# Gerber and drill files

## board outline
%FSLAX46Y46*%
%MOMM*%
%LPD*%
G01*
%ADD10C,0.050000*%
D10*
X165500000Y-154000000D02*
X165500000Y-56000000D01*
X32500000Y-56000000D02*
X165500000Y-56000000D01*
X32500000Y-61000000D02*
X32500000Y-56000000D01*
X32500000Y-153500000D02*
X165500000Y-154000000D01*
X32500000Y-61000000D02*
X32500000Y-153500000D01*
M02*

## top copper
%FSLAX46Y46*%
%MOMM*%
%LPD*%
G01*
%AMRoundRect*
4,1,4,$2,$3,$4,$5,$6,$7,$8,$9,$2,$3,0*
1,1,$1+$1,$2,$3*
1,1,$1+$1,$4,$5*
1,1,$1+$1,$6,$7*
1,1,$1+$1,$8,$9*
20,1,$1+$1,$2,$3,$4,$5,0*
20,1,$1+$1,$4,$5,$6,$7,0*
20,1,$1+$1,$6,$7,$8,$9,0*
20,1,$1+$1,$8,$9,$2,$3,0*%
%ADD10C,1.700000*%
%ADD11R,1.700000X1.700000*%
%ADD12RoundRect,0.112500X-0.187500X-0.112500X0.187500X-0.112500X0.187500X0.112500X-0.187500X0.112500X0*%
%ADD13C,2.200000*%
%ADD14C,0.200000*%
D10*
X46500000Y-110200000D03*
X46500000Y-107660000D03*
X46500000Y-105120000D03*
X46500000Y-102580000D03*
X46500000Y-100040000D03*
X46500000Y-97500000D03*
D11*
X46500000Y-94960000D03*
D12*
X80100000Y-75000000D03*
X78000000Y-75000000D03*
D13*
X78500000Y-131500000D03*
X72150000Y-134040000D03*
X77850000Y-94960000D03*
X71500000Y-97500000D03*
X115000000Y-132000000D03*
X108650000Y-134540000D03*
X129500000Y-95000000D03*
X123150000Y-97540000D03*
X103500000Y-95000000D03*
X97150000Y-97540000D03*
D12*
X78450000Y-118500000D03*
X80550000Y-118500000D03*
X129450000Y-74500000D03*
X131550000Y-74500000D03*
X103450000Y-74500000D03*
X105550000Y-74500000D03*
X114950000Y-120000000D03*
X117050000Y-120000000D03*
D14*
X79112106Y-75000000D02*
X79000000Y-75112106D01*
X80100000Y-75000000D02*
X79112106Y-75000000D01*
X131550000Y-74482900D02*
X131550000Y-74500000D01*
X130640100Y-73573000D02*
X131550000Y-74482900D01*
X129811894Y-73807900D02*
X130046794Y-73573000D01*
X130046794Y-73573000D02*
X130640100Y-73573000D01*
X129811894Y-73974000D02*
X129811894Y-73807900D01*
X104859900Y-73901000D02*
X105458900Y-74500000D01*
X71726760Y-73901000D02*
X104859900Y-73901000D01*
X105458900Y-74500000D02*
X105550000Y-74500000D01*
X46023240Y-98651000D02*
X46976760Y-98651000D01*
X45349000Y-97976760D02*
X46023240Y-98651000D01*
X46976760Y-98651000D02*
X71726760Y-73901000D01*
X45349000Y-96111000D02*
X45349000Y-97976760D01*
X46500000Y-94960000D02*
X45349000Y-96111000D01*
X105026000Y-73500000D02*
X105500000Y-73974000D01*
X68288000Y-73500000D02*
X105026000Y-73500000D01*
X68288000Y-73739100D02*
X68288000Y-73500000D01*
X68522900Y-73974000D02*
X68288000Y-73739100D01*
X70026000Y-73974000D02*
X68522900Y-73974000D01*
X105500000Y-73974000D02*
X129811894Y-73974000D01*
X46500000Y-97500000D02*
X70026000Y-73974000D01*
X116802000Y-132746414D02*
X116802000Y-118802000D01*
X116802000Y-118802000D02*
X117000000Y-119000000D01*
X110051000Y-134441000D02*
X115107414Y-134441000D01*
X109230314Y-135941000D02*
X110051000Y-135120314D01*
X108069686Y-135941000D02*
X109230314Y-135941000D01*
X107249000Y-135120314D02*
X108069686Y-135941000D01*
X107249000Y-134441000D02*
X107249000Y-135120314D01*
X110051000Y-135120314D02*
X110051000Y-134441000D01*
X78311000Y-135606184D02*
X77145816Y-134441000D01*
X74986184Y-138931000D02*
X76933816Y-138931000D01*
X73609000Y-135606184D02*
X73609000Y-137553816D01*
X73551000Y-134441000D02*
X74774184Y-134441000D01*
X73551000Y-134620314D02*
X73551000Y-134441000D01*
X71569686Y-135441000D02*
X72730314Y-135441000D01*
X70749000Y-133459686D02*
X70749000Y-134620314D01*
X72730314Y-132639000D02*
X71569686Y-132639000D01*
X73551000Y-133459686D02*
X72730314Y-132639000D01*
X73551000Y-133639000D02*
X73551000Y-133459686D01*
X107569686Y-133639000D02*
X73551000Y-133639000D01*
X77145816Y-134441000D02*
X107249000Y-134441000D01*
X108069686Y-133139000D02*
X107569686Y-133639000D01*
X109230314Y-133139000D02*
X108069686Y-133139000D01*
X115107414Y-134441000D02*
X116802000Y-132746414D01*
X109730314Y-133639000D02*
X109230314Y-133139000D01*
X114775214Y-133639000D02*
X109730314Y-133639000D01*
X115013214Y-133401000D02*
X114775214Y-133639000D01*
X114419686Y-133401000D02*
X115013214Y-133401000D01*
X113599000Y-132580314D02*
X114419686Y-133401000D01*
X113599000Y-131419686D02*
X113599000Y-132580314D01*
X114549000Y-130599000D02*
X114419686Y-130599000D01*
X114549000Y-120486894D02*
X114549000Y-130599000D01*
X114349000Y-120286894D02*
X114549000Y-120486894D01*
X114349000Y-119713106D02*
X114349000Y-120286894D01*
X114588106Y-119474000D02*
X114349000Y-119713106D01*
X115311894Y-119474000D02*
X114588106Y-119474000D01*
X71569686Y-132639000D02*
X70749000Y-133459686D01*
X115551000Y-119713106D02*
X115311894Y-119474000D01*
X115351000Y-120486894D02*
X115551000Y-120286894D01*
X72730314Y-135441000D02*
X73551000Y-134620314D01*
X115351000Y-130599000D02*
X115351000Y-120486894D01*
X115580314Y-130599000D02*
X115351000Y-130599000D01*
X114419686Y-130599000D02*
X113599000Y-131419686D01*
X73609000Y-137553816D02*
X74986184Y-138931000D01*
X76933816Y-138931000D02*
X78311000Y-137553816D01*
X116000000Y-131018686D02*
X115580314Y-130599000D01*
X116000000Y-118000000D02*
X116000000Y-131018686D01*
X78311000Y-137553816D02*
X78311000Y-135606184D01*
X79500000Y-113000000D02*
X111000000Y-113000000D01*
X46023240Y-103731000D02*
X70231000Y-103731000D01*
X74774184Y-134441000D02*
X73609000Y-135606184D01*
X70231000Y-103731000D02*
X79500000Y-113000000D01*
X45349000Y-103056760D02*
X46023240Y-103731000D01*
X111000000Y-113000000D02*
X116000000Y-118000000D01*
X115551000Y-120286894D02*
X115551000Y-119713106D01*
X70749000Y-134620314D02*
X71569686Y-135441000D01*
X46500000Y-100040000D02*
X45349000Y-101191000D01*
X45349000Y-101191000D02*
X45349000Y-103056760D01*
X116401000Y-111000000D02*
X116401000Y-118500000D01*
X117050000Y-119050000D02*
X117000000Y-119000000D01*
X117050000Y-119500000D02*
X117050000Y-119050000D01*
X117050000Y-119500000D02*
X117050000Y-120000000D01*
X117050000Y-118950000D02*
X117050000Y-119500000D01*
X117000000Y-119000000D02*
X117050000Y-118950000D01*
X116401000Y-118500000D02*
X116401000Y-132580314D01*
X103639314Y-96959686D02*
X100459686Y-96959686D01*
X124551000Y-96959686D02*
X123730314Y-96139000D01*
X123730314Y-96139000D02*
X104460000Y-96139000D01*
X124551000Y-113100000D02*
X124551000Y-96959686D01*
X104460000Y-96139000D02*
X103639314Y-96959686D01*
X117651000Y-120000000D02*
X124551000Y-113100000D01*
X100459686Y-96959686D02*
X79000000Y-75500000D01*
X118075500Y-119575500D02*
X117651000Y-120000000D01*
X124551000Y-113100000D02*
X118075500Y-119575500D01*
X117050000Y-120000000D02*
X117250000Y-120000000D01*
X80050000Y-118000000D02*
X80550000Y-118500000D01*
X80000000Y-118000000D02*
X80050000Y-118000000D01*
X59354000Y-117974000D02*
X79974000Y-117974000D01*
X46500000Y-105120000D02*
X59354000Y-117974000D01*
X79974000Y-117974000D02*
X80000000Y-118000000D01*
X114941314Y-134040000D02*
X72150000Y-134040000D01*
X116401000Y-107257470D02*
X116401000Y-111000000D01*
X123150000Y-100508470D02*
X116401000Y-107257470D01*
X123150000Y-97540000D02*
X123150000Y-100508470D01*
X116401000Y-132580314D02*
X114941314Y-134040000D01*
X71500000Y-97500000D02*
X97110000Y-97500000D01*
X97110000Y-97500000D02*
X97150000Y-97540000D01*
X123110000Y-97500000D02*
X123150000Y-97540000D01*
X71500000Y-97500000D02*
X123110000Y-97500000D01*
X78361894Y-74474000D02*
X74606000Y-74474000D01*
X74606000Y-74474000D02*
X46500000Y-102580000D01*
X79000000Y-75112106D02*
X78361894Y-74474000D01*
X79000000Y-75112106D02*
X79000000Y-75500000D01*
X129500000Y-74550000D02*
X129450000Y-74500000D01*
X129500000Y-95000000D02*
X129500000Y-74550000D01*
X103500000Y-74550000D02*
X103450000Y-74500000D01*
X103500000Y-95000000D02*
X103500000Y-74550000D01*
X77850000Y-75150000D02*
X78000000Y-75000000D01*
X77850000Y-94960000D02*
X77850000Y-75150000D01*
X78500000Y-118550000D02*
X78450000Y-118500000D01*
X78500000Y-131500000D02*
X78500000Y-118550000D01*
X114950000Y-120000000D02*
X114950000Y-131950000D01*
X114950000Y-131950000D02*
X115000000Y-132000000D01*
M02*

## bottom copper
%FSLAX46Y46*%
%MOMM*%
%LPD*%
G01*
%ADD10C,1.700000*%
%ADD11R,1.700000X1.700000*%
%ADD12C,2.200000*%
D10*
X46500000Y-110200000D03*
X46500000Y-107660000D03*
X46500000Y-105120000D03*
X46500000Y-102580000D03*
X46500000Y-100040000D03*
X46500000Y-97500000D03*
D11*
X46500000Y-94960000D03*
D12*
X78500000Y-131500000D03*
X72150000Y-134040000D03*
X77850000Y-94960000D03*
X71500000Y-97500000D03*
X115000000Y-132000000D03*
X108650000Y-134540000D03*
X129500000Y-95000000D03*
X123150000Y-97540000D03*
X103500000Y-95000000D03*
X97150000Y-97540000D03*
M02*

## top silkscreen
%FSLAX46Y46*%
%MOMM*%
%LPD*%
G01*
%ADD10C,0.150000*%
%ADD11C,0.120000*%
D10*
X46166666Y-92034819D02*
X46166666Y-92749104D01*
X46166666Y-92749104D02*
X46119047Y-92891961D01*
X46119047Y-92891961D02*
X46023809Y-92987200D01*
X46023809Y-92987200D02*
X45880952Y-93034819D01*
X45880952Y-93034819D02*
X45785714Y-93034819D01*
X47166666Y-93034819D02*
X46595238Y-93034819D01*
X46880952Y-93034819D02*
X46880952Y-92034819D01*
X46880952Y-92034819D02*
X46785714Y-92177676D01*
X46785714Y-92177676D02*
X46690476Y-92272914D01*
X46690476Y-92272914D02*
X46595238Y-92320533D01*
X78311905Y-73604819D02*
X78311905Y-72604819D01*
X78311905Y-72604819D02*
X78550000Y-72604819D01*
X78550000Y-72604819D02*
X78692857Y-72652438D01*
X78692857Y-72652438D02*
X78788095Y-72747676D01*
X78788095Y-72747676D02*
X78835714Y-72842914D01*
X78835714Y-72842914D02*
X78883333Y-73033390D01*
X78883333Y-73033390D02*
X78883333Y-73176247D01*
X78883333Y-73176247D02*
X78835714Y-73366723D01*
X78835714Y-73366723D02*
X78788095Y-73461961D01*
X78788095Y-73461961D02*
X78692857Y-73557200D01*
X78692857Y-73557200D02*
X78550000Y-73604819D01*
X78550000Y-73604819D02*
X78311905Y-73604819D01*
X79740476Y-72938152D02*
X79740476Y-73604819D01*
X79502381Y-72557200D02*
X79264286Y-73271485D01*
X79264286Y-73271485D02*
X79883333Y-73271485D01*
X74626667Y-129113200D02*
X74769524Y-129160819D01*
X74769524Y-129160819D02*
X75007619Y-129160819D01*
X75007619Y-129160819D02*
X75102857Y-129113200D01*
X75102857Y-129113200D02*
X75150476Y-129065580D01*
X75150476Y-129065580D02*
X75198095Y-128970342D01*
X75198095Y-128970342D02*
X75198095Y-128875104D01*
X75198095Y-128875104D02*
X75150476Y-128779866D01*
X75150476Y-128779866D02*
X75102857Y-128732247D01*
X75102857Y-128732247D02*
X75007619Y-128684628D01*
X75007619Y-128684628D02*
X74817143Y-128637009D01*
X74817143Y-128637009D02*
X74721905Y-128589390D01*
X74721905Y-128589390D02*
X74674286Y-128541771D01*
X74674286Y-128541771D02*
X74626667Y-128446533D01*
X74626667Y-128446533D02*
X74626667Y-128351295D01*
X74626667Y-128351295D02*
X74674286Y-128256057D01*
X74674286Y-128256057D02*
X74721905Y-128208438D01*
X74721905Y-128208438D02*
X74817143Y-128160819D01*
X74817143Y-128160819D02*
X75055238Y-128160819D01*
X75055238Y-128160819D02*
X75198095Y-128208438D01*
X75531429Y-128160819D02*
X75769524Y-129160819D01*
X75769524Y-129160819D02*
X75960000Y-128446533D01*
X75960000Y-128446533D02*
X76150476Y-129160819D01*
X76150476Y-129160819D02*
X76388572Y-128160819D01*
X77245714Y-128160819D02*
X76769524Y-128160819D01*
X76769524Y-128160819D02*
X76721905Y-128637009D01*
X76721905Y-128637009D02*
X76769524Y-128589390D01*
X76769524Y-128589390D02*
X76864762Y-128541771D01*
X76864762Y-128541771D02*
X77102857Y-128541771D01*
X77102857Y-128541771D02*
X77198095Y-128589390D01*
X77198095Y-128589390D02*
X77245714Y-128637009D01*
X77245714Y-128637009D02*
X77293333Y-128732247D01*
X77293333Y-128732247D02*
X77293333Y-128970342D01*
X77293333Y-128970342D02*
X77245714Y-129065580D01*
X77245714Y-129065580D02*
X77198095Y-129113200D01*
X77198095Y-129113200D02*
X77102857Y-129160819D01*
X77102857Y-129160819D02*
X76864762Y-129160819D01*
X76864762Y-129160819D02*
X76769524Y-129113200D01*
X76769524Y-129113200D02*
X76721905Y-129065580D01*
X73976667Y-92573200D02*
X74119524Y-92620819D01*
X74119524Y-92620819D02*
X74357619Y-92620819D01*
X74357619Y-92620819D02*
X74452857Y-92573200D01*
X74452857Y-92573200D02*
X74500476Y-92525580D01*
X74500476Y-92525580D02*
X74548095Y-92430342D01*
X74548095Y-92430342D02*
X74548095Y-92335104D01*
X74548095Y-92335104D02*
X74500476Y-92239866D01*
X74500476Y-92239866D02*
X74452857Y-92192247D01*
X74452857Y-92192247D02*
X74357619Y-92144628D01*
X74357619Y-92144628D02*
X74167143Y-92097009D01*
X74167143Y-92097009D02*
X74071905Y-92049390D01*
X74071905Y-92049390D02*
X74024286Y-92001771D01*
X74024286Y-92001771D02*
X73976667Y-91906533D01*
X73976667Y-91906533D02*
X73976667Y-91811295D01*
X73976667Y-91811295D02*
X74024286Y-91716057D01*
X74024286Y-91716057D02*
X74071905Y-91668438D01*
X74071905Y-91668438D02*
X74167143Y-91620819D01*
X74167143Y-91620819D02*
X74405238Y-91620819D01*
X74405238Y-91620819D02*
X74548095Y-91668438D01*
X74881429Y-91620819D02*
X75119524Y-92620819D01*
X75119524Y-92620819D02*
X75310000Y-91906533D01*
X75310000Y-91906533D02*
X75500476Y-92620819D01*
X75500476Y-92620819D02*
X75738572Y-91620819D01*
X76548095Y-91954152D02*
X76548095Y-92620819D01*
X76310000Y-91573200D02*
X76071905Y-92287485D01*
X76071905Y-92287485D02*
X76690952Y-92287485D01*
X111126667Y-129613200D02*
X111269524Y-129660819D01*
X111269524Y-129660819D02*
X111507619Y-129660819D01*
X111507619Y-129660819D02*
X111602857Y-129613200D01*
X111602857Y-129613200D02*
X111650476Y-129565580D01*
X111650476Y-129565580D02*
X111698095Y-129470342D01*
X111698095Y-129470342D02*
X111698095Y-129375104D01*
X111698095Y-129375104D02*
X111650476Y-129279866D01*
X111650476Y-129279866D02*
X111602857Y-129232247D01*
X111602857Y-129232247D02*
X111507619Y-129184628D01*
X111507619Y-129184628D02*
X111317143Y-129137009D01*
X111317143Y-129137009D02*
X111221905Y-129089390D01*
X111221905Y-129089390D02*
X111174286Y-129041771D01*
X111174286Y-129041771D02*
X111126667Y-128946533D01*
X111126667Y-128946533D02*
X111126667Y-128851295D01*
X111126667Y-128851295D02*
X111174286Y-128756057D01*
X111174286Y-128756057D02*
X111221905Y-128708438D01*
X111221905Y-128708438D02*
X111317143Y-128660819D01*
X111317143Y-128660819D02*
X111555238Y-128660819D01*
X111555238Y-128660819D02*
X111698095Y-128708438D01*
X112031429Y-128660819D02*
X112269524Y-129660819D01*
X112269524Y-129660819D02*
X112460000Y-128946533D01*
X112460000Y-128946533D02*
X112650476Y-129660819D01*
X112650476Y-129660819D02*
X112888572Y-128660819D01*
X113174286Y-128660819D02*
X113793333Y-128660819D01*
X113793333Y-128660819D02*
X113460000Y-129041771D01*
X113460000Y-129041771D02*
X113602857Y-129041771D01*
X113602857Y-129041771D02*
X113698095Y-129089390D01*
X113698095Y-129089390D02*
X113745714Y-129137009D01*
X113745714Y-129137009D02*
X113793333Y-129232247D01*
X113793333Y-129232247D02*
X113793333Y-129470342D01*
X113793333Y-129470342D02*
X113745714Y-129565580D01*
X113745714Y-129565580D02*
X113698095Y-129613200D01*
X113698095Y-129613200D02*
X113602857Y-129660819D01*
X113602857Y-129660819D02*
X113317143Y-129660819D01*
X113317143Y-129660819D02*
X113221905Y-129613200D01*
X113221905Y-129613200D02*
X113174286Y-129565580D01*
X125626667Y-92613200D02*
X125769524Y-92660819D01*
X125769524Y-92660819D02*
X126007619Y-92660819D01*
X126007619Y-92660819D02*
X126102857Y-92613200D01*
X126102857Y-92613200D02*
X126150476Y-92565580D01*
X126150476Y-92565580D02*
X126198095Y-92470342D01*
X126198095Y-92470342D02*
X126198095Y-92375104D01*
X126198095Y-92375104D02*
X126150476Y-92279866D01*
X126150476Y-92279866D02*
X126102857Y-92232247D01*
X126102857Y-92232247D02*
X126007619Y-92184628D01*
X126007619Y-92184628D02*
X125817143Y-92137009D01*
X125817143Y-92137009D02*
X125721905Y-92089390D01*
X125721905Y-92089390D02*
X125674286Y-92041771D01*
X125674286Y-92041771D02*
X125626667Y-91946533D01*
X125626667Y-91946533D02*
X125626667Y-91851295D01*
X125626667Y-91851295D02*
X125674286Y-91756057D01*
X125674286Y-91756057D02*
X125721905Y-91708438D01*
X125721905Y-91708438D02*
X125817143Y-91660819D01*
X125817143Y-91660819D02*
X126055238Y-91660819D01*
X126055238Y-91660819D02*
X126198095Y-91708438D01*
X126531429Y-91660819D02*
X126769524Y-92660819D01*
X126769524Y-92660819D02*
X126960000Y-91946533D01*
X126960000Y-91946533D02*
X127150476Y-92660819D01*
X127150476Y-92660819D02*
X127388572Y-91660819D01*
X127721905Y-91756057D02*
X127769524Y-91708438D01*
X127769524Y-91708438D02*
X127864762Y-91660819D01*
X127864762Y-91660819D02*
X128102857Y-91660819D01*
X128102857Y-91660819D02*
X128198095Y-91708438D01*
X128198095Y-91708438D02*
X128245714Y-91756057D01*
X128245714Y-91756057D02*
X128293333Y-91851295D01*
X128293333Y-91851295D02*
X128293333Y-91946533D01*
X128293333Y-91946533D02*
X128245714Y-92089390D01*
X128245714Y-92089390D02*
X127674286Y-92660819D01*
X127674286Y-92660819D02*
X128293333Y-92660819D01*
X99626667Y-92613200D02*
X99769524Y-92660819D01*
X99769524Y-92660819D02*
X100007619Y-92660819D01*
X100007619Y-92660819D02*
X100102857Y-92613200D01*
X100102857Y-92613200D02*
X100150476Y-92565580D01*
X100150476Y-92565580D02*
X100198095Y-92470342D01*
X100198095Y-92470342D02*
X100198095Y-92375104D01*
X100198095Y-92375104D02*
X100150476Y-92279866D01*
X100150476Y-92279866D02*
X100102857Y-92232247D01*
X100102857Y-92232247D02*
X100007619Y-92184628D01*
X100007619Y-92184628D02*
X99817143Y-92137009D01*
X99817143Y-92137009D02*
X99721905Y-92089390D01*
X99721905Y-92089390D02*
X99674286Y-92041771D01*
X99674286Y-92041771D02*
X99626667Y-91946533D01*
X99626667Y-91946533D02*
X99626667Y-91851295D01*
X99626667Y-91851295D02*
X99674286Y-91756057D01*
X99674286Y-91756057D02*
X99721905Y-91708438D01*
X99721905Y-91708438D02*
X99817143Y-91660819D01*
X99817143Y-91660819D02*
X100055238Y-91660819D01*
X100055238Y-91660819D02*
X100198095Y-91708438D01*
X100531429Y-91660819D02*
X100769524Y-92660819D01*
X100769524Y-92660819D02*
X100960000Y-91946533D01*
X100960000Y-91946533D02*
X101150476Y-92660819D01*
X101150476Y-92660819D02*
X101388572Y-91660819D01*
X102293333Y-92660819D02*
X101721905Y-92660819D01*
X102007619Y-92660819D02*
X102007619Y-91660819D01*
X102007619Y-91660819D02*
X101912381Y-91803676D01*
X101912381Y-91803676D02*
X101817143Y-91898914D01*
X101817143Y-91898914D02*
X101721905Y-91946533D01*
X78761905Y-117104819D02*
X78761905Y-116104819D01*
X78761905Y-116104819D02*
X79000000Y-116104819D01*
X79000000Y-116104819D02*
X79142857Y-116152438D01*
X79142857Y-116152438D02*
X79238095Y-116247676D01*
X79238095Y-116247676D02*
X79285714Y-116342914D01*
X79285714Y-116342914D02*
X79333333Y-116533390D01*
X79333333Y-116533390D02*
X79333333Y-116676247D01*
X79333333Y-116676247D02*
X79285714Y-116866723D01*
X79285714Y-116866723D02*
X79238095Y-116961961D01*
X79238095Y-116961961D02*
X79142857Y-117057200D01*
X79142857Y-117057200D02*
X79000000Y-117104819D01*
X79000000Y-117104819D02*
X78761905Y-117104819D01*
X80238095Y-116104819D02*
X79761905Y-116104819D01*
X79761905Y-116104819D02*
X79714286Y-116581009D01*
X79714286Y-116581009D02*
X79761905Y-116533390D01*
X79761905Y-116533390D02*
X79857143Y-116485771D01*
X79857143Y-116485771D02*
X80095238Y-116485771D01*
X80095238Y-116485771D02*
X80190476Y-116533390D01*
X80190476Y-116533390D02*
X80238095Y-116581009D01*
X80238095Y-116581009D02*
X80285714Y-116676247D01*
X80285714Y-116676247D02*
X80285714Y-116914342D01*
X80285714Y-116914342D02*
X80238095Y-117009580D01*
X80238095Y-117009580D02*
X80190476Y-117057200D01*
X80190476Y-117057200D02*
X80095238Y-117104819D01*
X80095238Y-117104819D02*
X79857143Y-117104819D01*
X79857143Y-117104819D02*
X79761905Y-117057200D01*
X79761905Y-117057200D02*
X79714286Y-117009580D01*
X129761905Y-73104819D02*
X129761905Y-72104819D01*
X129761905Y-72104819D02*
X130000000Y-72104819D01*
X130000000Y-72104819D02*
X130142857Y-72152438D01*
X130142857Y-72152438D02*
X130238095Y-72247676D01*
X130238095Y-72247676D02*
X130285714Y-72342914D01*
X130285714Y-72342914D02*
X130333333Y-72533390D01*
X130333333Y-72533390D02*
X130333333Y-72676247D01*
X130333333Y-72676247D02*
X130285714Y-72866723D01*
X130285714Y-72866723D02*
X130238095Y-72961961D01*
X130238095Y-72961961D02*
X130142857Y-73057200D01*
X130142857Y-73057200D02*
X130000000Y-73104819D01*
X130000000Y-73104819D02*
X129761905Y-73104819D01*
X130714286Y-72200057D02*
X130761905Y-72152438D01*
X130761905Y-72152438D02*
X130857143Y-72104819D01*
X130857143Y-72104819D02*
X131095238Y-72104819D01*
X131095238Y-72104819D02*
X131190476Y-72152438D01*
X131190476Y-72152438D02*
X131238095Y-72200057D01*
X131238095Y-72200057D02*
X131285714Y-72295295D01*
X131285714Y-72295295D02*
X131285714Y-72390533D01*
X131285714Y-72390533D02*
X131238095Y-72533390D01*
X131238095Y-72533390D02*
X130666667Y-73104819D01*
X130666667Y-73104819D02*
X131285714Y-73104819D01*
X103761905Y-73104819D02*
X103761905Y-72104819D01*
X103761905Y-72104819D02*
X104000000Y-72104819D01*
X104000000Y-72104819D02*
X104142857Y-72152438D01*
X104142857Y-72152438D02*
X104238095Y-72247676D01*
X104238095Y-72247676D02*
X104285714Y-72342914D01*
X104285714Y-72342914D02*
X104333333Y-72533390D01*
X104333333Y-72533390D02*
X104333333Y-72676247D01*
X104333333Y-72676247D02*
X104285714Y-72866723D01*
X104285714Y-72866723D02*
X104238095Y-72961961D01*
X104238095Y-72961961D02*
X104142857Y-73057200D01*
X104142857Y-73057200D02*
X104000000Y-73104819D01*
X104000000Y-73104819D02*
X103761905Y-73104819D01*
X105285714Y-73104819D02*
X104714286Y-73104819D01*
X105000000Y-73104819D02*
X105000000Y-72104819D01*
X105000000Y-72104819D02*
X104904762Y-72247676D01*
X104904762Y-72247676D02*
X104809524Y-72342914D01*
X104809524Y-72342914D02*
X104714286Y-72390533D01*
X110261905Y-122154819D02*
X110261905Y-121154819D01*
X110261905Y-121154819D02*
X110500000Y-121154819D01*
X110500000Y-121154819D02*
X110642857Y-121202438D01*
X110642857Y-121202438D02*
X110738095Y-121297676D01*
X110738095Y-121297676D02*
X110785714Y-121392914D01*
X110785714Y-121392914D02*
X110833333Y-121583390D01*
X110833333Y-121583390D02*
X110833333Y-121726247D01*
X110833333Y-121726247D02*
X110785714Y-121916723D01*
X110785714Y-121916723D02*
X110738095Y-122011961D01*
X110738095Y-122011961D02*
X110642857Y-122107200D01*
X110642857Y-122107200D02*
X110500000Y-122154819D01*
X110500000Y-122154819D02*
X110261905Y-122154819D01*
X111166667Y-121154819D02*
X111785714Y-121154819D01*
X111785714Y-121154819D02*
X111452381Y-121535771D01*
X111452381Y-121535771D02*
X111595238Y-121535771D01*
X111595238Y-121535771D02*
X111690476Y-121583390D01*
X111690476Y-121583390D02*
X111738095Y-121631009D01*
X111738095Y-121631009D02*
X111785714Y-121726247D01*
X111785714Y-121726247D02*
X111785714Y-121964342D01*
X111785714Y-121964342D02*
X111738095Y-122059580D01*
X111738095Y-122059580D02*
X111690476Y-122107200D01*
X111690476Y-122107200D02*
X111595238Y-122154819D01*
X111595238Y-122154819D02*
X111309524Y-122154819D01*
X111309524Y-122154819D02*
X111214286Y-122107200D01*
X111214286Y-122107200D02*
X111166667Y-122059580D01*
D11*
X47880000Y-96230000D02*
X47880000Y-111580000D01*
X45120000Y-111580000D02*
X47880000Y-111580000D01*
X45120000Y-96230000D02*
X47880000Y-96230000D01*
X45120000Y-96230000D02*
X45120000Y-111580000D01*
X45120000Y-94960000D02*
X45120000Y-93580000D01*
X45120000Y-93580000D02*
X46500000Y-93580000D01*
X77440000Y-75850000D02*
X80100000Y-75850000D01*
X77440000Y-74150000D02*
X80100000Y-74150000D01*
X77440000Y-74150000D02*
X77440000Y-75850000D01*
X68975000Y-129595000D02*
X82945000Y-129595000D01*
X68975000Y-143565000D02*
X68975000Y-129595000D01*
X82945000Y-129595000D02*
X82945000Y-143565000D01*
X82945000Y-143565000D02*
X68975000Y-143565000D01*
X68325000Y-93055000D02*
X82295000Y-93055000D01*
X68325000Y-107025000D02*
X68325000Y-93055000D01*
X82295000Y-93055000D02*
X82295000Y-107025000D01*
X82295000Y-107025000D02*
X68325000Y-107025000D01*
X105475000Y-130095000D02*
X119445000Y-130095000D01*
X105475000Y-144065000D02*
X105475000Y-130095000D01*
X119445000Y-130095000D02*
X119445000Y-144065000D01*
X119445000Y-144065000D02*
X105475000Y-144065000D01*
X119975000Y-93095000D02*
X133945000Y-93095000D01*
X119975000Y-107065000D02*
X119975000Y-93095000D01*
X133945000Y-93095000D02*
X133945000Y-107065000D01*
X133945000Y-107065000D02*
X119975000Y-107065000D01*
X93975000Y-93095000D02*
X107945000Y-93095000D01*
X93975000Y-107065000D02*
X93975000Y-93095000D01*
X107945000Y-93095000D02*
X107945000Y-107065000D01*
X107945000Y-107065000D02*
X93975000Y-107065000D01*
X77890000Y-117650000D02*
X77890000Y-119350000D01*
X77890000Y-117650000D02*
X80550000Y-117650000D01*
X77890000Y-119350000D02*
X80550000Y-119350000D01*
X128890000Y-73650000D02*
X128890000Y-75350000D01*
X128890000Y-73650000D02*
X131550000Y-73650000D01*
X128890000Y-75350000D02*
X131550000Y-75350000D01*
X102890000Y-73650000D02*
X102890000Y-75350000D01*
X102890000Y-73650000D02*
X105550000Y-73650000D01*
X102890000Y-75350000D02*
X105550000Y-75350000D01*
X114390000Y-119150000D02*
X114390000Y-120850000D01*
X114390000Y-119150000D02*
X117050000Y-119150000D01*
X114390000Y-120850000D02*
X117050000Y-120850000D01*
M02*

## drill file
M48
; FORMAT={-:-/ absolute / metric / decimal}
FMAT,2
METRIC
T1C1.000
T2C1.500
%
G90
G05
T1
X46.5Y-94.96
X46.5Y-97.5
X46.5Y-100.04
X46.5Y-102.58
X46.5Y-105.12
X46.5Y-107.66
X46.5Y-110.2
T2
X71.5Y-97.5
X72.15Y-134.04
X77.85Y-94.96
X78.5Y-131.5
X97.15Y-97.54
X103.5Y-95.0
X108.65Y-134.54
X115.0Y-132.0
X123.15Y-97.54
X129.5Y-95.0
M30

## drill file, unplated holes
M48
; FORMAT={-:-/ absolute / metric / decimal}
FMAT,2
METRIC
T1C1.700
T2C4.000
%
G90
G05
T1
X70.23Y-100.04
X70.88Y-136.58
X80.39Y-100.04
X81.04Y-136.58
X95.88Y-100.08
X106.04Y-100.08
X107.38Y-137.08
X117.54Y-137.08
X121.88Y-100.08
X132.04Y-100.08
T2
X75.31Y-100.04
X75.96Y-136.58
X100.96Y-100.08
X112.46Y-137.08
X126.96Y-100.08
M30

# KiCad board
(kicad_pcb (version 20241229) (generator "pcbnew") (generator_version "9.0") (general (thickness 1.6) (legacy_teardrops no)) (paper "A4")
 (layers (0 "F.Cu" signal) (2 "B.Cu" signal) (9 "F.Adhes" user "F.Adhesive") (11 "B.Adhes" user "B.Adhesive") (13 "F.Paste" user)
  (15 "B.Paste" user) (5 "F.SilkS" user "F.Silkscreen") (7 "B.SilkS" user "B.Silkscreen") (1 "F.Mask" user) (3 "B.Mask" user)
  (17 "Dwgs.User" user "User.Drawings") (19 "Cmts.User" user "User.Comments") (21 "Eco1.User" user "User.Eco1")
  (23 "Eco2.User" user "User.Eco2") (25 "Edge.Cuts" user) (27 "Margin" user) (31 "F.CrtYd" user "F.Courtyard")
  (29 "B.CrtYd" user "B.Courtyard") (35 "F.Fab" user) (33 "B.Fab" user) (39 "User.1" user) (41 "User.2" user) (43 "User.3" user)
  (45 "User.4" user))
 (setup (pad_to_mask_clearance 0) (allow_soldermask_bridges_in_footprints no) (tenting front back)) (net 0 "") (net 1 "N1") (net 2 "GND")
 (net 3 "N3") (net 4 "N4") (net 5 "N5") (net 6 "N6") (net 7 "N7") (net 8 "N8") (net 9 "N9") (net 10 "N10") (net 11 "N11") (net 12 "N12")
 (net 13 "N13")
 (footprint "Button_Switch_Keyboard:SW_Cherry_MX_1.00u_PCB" (layer "F.Cu") (at 77.85 94.96)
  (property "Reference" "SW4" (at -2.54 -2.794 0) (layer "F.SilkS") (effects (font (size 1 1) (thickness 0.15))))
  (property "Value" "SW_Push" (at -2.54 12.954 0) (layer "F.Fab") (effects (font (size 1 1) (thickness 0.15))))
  (fp_line (start -9.525 -1.905) (end 4.445 -1.905) (stroke (width 0.12) (type solid)) (layer "F.SilkS"))
  (fp_line (start -9.525 12.065) (end -9.525 -1.905) (stroke (width 0.12) (type solid)) (layer "F.SilkS"))
  (fp_line (start 4.445 -1.905) (end 4.445 12.065) (stroke (width 0.12) (type solid)) (layer "F.SilkS"))
  (fp_line (start 4.445 12.065) (end -9.525 12.065) (stroke (width 0.12) (type solid)) (layer "F.SilkS"))
  (pad "" np_thru_hole circle (at -7.62 5.08) (size 1.7 1.7) (drill 1.7) (layers "*.Cu" "*.Mask"))
  (pad "" np_thru_hole circle (at -2.54 5.08) (size 4 4) (drill 4) (layers "*.Cu" "*.Mask"))
  (pad "" np_thru_hole circle (at 2.54 5.08) (size 1.7 1.7) (drill 1.7) (layers "*.Cu" "*.Mask"))
  (pad "1" thru_hole circle (at 0 0) (size 2.2 2.2) (drill 1.5) (layers "*.Cu" "*.Mask") (remove_unused_layers no) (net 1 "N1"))
  (pad "2" thru_hole circle (at -6.35 2.54) (size 2.2 2.2) (drill 1.5) (layers "*.Cu" "*.Mask") (remove_unused_layers no) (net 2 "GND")))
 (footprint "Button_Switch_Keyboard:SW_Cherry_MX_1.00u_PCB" (layer "F.Cu") (at 115 132)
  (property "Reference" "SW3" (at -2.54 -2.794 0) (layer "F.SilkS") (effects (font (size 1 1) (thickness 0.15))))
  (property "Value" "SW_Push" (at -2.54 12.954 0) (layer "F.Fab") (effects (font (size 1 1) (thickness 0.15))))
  (fp_line (start -9.525 -1.905) (end 4.445 -1.905) (stroke (width 0.12) (type solid)) (layer "F.SilkS"))
  (fp_line (start -9.525 12.065) (end -9.525 -1.905) (stroke (width 0.12) (type solid)) (layer "F.SilkS"))
  (fp_line (start 4.445 -1.905) (end 4.445 12.065) (stroke (width 0.12) (type solid)) (layer "F.SilkS"))
  (fp_line (start 4.445 12.065) (end -9.525 12.065) (stroke (width 0.12) (type solid)) (layer "F.SilkS"))
  (pad "" np_thru_hole circle (at -7.62 5.08) (size 1.7 1.7) (drill 1.7) (layers "*.Cu" "*.Mask"))
  (pad "" np_thru_hole circle (at -2.54 5.08) (size 4 4) (drill 4) (layers "*.Cu" "*.Mask"))
  (pad "" np_thru_hole circle (at 2.54 5.08) (size 1.7 1.7) (drill 1.7) (layers "*.Cu" "*.Mask"))
  (pad "1" thru_hole circle (at 0 0) (size 2.2 2.2) (drill 1.5) (layers "*.Cu" "*.Mask") (remove_unused_layers no) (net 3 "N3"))
  (pad "2" thru_hole circle (at -6.35 2.54) (size 2.2 2.2) (drill 1.5) (layers "*.Cu" "*.Mask") (remove_unused_layers no) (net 2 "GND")))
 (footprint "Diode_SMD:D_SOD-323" (layer "F.Cu") (at 79.05 75)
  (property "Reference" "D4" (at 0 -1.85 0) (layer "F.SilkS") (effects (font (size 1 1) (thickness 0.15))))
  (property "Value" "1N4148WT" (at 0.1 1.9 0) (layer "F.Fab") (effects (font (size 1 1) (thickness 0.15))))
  (fp_line (start -1.61 -0.85) (end -1.61 0.85) (stroke (width 0.12) (type solid)) (layer "F.SilkS"))
  (fp_line (start -1.61 -0.85) (end 1.05 -0.85) (stroke (width 0.12) (type solid)) (layer "F.SilkS"))
  (fp_line (start -1.61 0.85) (end 1.05 0.85) (stroke (width 0.12) (type solid)) (layer "F.SilkS"))
  (pad "1" smd roundrect (at -1.05 0) (size 0.6 0.45) (layers "F.Cu" "F.Mask" "F.Paste") (roundrect_rratio 0.25) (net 1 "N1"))
  (pad "2" smd roundrect (at 1.05 0) (size 0.6 0.45) (layers "F.Cu" "F.Mask" "F.Paste") (roundrect_rratio 0.25) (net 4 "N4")))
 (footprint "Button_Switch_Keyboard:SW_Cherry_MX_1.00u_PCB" (layer "F.Cu") (at 78.5 131.5)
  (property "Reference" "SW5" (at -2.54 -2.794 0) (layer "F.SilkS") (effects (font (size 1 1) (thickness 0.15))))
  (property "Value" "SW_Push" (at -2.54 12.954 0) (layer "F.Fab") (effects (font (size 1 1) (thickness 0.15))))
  (fp_line (start -9.525 -1.905) (end 4.445 -1.905) (stroke (width 0.12) (type solid)) (layer "F.SilkS"))
  (fp_line (start -9.525 12.065) (end -9.525 -1.905) (stroke (width 0.12) (type solid)) (layer "F.SilkS"))
  (fp_line (start 4.445 -1.905) (end 4.445 12.065) (stroke (width 0.12) (type solid)) (layer "F.SilkS"))
  (fp_line (start 4.445 12.065) (end -9.525 12.065) (stroke (width 0.12) (type solid)) (layer "F.SilkS"))
  (pad "" np_thru_hole circle (at -7.62 5.08) (size 1.7 1.7) (drill 1.7) (layers "*.Cu" "*.Mask"))
  (pad "" np_thru_hole circle (at -2.54 5.08) (size 4 4) (drill 4) (layers "*.Cu" "*.Mask"))
  (pad "" np_thru_hole circle (at 2.54 5.08) (size 1.7 1.7) (drill 1.7) (layers "*.Cu" "*.Mask"))
  (pad "1" thru_hole circle (at 0 0) (size 2.2 2.2) (drill 1.5) (layers "*.Cu" "*.Mask") (remove_unused_layers no) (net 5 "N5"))
  (pad "2" thru_hole circle (at -6.35 2.54) (size 2.2 2.2) (drill 1.5) (layers "*.Cu" "*.Mask") (remove_unused_layers no) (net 2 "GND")))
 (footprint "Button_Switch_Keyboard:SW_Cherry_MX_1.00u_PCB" (layer "F.Cu") (at 103.5 95)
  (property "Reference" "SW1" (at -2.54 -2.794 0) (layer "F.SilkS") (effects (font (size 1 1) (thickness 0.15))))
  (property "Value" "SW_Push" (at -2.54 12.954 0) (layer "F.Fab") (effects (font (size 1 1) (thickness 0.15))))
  (fp_line (start -9.525 -1.905) (end 4.445 -1.905) (stroke (width 0.12) (type solid)) (layer "F.SilkS"))
  (fp_line (start -9.525 12.065) (end -9.525 -1.905) (stroke (width 0.12) (type solid)) (layer "F.SilkS"))
  (fp_line (start 4.445 -1.905) (end 4.445 12.065) (stroke (width 0.12) (type solid)) (layer "F.SilkS"))
  (fp_line (start 4.445 12.065) (end -9.525 12.065) (stroke (width 0.12) (type solid)) (layer "F.SilkS"))
  (pad "" np_thru_hole circle (at -7.62 5.08) (size 1.7 1.7) (drill 1.7) (layers "*.Cu" "*.Mask"))
  (pad "" np_thru_hole circle (at -2.54 5.08) (size 4 4) (drill 4) (layers "*.Cu" "*.Mask"))
  (pad "" np_thru_hole circle (at 2.54 5.08) (size 1.7 1.7) (drill 1.7) (layers "*.Cu" "*.Mask"))
  (pad "1" thru_hole circle (at 0 0) (size 2.2 2.2) (drill 1.5) (layers "*.Cu" "*.Mask") (remove_unused_layers no) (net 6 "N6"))
  (pad "2" thru_hole circle (at -6.35 2.54) (size 2.2 2.2) (drill 1.5) (layers "*.Cu" "*.Mask") (remove_unused_layers no) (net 2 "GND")))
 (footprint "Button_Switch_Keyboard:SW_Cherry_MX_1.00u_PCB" (layer "F.Cu") (at 129.5 95)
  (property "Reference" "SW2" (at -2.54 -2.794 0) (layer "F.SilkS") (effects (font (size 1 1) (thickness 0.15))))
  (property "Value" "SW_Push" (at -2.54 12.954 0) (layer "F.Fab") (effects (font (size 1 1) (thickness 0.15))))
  (fp_line (start -9.525 -1.905) (end 4.445 -1.905) (stroke (width 0.12) (type solid)) (layer "F.SilkS"))
  (fp_line (start -9.525 12.065) (end -9.525 -1.905) (stroke (width 0.12) (type solid)) (layer "F.SilkS"))
  (fp_line (start 4.445 -1.905) (end 4.445 12.065) (stroke (width 0.12) (type solid)) (layer "F.SilkS"))
  (fp_line (start 4.445 12.065) (end -9.525 12.065) (stroke (width 0.12) (type solid)) (layer "F.SilkS"))
  (pad "" np_thru_hole circle (at -7.62 5.08) (size 1.7 1.7) (drill 1.7) (layers "*.Cu" "*.Mask"))
  (pad "" np_thru_hole circle (at -2.54 5.08) (size 4 4) (drill 4) (layers "*.Cu" "*.Mask"))
  (pad "" np_thru_hole circle (at 2.54 5.08) (size 1.7 1.7) (drill 1.7) (layers "*.Cu" "*.Mask"))
  (pad "1" thru_hole circle (at 0 0) (size 2.2 2.2) (drill 1.5) (layers "*.Cu" "*.Mask") (remove_unused_layers no) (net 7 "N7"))
  (pad "2" thru_hole circle (at -6.35 2.54) (size 2.2 2.2) (drill 1.5) (layers "*.Cu" "*.Mask") (remove_unused_layers no) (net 2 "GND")))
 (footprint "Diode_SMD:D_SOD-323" (layer "F.Cu") (at 79.5 118.5)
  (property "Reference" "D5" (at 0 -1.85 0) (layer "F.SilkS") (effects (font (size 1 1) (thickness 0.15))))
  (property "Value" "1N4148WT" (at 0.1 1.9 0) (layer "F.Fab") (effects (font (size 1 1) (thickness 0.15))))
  (fp_line (start -1.61 -0.85) (end -1.61 0.85) (stroke (width 0.12) (type solid)) (layer "F.SilkS"))
  (fp_line (start -1.61 -0.85) (end 1.05 -0.85) (stroke (width 0.12) (type solid)) (layer "F.SilkS"))
  (fp_line (start -1.61 0.85) (end 1.05 0.85) (stroke (width 0.12) (type solid)) (layer "F.SilkS"))
  (pad "1" smd roundrect (at -1.05 0) (size 0.6 0.45) (layers "F.Cu" "F.Mask" "F.Paste") (roundrect_rratio 0.25) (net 5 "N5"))
  (pad "2" smd roundrect (at 1.05 0) (size 0.6 0.45) (layers "F.Cu" "F.Mask" "F.Paste") (roundrect_rratio 0.25) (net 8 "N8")))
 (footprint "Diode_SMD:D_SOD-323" (layer "F.Cu") (at 130.5 74.5)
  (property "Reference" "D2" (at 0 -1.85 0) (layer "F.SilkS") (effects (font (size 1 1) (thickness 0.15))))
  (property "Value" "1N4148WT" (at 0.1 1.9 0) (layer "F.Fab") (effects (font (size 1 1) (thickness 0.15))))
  (fp_line (start -1.61 -0.85) (end -1.61 0.85) (stroke (width 0.12) (type solid)) (layer "F.SilkS"))
  (fp_line (start -1.61 -0.85) (end 1.05 -0.85) (stroke (width 0.12) (type solid)) (layer "F.SilkS"))
  (fp_line (start -1.61 0.85) (end 1.05 0.85) (stroke (width 0.12) (type solid)) (layer "F.SilkS"))
  (pad "1" smd roundrect (at -1.05 0) (size 0.6 0.45) (layers "F.Cu" "F.Mask" "F.Paste") (roundrect_rratio 0.25) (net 7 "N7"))
  (pad "2" smd roundrect (at 1.05 0) (size 0.6 0.45) (layers "F.Cu" "F.Mask" "F.Paste") (roundrect_rratio 0.25) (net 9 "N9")))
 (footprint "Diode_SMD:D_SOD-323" (layer "F.Cu") (at 104.5 74.5)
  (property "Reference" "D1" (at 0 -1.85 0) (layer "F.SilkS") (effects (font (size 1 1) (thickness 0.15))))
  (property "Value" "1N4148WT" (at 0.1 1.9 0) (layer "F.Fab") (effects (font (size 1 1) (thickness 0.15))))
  (fp_line (start -1.61 -0.85) (end -1.61 0.85) (stroke (width 0.12) (type solid)) (layer "F.SilkS"))
  (fp_line (start -1.61 -0.85) (end 1.05 -0.85) (stroke (width 0.12) (type solid)) (layer "F.SilkS"))
  (fp_line (start -1.61 0.85) (end 1.05 0.85) (stroke (width 0.12) (type solid)) (layer "F.SilkS"))
  (pad "1" smd roundrect (at -1.05 0) (size 0.6 0.45) (layers "F.Cu" "F.Mask" "F.Paste") (roundrect_rratio 0.25) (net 6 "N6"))
  (pad "2" smd roundrect (at 1.05 0) (size 0.6 0.45) (layers "F.Cu" "F.Mask" "F.Paste") (roundrect_rratio 0.25) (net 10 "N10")))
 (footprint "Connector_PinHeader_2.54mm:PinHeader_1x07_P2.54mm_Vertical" (layer "F.Cu") (at 46.5 94.96)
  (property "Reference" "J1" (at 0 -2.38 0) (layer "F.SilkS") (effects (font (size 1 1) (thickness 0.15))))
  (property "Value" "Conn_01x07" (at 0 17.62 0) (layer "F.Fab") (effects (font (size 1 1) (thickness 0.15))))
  (fp_line (start -1.38 -1.38) (end 0 -1.38) (stroke (width 0.12) (type solid)) (layer "F.SilkS"))
  (fp_line (start -1.38 0) (end -1.38 -1.38) (stroke (width 0.12) (type solid)) (layer "F.SilkS"))
  (fp_line (start -1.38 1.27) (end -1.38 16.62) (stroke (width 0.12) (type solid)) (layer "F.SilkS"))
  (fp_line (start -1.38 1.27) (end 1.38 1.27) (stroke (width 0.12) (type solid)) (layer "F.SilkS"))
  (fp_line (start -1.38 16.62) (end 1.38 16.62) (stroke (width 0.12) (type solid)) (layer "F.SilkS"))
  (fp_line (start 1.38 1.27) (end 1.38 16.62) (stroke (width 0.12) (type solid)) (layer "F.SilkS"))
  (pad "1" thru_hole rect (at 0 0) (size 1.7 1.7) (drill 1) (layers "*.Cu" "*.Mask") (remove_unused_layers no) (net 10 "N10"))
  (pad "2" thru_hole circle (at 0 2.54) (size 1.7 1.7) (drill 1) (layers "*.Cu" "*.Mask") (remove_unused_layers no) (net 9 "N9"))
  (pad "3" thru_hole circle (at 0 5.08) (size 1.7 1.7) (drill 1) (layers "*.Cu" "*.Mask") (remove_unused_layers no) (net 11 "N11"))
  (pad "4" thru_hole circle (at 0 7.62) (size 1.7 1.7) (drill 1) (layers "*.Cu" "*.Mask") (remove_unused_layers no) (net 4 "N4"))
  (pad "5" thru_hole circle (at 0 10.16) (size 1.7 1.7) (drill 1) (layers "*.Cu" "*.Mask") (remove_unused_layers no) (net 8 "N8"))
  (pad "6" thru_hole circle (at 0 12.7) (size 1.7 1.7) (drill 1) (layers "*.Cu" "*.Mask") (remove_unused_layers no) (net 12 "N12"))
  (pad "7" thru_hole circle (at 0 15.24) (size 1.7 1.7) (drill 1) (layers "*.Cu" "*.Mask") (remove_unused_layers no) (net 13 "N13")))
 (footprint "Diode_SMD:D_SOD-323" (layer "F.Cu") (at 116 120)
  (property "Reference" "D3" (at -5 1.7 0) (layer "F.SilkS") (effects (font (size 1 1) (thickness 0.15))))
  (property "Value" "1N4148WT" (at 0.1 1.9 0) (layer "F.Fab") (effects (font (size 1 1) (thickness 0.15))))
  (fp_line (start -1.61 -0.85) (end -1.61 0.85) (stroke (width 0.12) (type solid)) (layer "F.SilkS"))
  (fp_line (start -1.61 -0.85) (end 1.05 -0.85) (stroke (width 0.12) (type solid)) (layer "F.SilkS"))
  (fp_line (start -1.61 0.85) (end 1.05 0.85) (stroke (width 0.12) (type solid)) (layer "F.SilkS"))
  (pad "1" smd roundrect (at -1.05 0) (size 0.6 0.45) (layers "F.Cu" "F.Mask" "F.Paste") (roundrect_rratio 0.25) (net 3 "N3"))
  (pad "2" smd roundrect (at 1.05 0) (size 0.6 0.45) (layers "F.Cu" "F.Mask" "F.Paste") (roundrect_rratio 0.25) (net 11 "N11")))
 (gr_line (start 32.5 61) (end 32.5 153.5) (stroke (width 0.05) (type default)) (layer "Edge.Cuts"))
 (gr_line (start 32.5 153.5) (end 165.5 154) (stroke (width 0.05) (type default)) (layer "Edge.Cuts"))
 (gr_line (start 165.5 154) (end 165.5 56) (stroke (width 0.05) (type default)) (layer "Edge.Cuts"))
 (gr_line (start 32.5 56) (end 165.5 56) (stroke (width 0.05) (type default)) (layer "Edge.Cuts"))
 (gr_line (start 32.5 61) (end 32.5 56) (stroke (width 0.05) (type default)) (layer "Edge.Cuts"))
 (segment (start 103.5 74.55) (end 103.45 74.5) (width 0.2) (layer "F.Cu") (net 6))
 (segment (start 103.5 95) (end 103.5 74.55) (width 0.2) (layer "F.Cu") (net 6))
 (segment (start 46.02324 98.651) (end 46.97676 98.651) (width 0.2) (layer "F.Cu") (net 10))
 (segment (start 45.349 96.111) (end 45.349 97.97676) (width 0.2) (layer "F.Cu") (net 10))
 (segment (start 104.8599 73.901) (end 105.4589 74.5) (width 0.2) (layer "F.Cu") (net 10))
 (segment (start 46.5 94.96) (end 45.349 96.111) (width 0.2) (layer "F.Cu") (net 10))
 (segment (start 105.4589 74.5) (end 105.55 74.5) (width 0.2) (layer "F.Cu") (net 10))
 (segment (start 45.349 97.97676) (end 46.02324 98.651) (width 0.2) (layer "F.Cu") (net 10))
 (segment (start 46.97676 98.651) (end 71.72676 73.901) (width 0.2) (layer "F.Cu") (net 10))
 (segment (start 71.72676 73.901) (end 104.8599 73.901) (width 0.2) (layer "F.Cu") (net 10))
 (segment (start 68.288 73.7391) (end 68.288 73.5) (width 0.2) (layer "F.Cu") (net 9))
 (segment (start 129.811894 73.974) (end 129.811894 73.8079) (width 0.2) (layer "F.Cu") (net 9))
 (segment (start 68.5229 73.974) (end 68.288 73.7391) (width 0.2) (layer "F.Cu") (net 9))
 (segment (start 131.55 74.4829) (end 131.55 74.5) (width 0.2) (layer "F.Cu") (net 9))
 (segment (start 68.288 73.5) (end 105.026 73.5) (width 0.2) (layer "F.Cu") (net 9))
 (segment (start 130.6401 73.573) (end 131.55 74.4829) (width 0.2) (layer "F.Cu") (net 9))
 (segment (start 70.026 73.974) (end 68.5229 73.974) (width 0.2) (layer "F.Cu") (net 9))
 (segment (start 105.026 73.5) (end 105.5 73.974) (width 0.2) (layer "F.Cu") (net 9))
 (segment (start 130.046794 73.573) (end 130.6401 73.573) (width 0.2) (layer "F.Cu") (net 9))
 (segment (start 46.5 97.5) (end 70.026 73.974) (width 0.2) (layer "F.Cu") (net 9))
 (segment (start 105.5 73.974) (end 129.811894 73.974) (width 0.2) (layer "F.Cu") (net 9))
 (segment (start 129.811894 73.8079) (end 130.046794 73.573) (width 0.2) (layer "F.Cu") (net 9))
 (segment (start 129.5 74.55) (end 129.45 74.5) (width 0.2) (layer "F.Cu") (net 7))
 (segment (start 129.5 95) (end 129.5 74.55) (width 0.2) (layer "F.Cu") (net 7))
 (segment (start 114.95 131.95) (end 115 132) (width 0.2) (layer "F.Cu") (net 3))
 (segment (start 114.95 120) (end 114.95 131.95) (width 0.2) (layer "F.Cu") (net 3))
 (segment (start 73.551 134.620314) (end 73.551 134.441) (width 0.2) (layer "F.Cu") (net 11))
 (segment (start 73.551 134.441) (end 74.774184 134.441) (width 0.2) (layer "F.Cu") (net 11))
 (segment (start 111 113) (end 116 118) (width 0.2) (layer "F.Cu") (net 11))
 (segment (start 76.933816 138.931) (end 78.311 137.553816) (width 0.2) (layer "F.Cu") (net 11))
 (segment (start 109.730314 133.639) (end 109.230314 133.139) (width 0.2) (layer "F.Cu") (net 11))
 (segment (start 46.02324 103.731) (end 70.231 103.731) (width 0.2) (layer "F.Cu") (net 11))
 (segment (start 109.230314 135.941) (end 110.051 135.120314) (width 0.2) (layer "F.Cu") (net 11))
 (segment (start 117.05 119.5) (end 117.05 120) (width 0.2) (layer "F.Cu") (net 11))
 (segment (start 70.749 134.620314) (end 71.569686 135.441) (width 0.2) (layer "F.Cu") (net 11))
 (segment (start 117.05 119.5) (end 117.05 119.05) (width 0.2) (layer "F.Cu") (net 11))
 (segment (start 107.249 135.120314) (end 108.069686 135.941) (width 0.2) (layer "F.Cu") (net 11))
 (segment (start 79.5 113) (end 111 113) (width 0.2) (layer "F.Cu") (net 11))
 (segment (start 109.230314 133.139) (end 108.069686 133.139) (width 0.2) (layer "F.Cu") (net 11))
 (segment (start 114.588106 119.474) (end 114.349 119.713106) (width 0.2) (layer "F.Cu") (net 11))
 (segment (start 116 118) (end 116 131.018686) (width 0.2) (layer "F.Cu") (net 11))
 (segment (start 116.802 118.802) (end 117 119) (width 0.2) (layer "F.Cu") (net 11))
 (segment (start 114.549 130.599) (end 114.419686 130.599) (width 0.2) (layer "F.Cu") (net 11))
 (segment (start 110.051 134.441) (end 115.107414 134.441) (width 0.2) (layer "F.Cu") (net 11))
 (segment (start 113.599 131.419686) (end 113.599 132.580314) (width 0.2) (layer "F.Cu") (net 11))
 (segment (start 70.231 103.731) (end 79.5 113) (width 0.2) (layer "F.Cu") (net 11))
 (segment (start 73.609 135.606184) (end 73.609 137.553816) (width 0.2) (layer "F.Cu") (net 11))
 (segment (start 115.107414 134.441) (end 116.802 132.746414) (width 0.2) (layer "F.Cu") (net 11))
 (segment (start 113.599 132.580314) (end 114.419686 133.401) (width 0.2) (layer "F.Cu") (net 11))
 (segment (start 115.013214 133.401) (end 114.775214 133.639) (width 0.2) (layer "F.Cu") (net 11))
 (segment (start 72.730314 132.639) (end 71.569686 132.639) (width 0.2) (layer "F.Cu") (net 11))
 (segment (start 115.311894 119.474) (end 114.588106 119.474) (width 0.2) (layer "F.Cu") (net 11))
 (segment (start 116 131.018686) (end 115.580314 130.599) (width 0.2) (layer "F.Cu") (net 11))
 (segment (start 107.569686 133.639) (end 73.551 133.639) (width 0.2) (layer "F.Cu") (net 11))
 (segment (start 72.730314 135.441) (end 73.551 134.620314) (width 0.2) (layer "F.Cu") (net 11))
 (segment (start 117.05 119.05) (end 117 119) (width 0.2) (layer "F.Cu") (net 11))
 (segment (start 115.580314 130.599) (end 115.351 130.599) (width 0.2) (layer "F.Cu") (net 11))
 (segment (start 117 119) (end 117.05 118.95) (width 0.2) (layer "F.Cu") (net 11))
 (segment (start 70.749 133.459686) (end 70.749 134.620314) (width 0.2) (layer "F.Cu") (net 11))
 (segment (start 117.05 118.95) (end 117.05 119.5) (width 0.2) (layer "F.Cu") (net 11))
 (segment (start 117.05 120) (end 117.25 120) (width 0.2) (layer "F.Cu") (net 11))
 (segment (start 45.349 103.05676) (end 46.02324 103.731) (width 0.2) (layer "F.Cu") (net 11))
 (segment (start 114.349 120.286894) (end 114.549 120.486894) (width 0.2) (layer "F.Cu") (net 11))
 (segment (start 114.775214 133.639) (end 109.730314 133.639) (width 0.2) (layer "F.Cu") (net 11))
 (segment (start 114.549 120.486894) (end 114.549 130.599) (width 0.2) (layer "F.Cu") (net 11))
 (segment (start 115.351 120.486894) (end 115.551 120.286894) (width 0.2) (layer "F.Cu") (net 11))
 (segment (start 108.069686 135.941) (end 109.230314 135.941) (width 0.2) (layer "F.Cu") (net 11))
 (segment (start 115.551 120.286894) (end 115.551 119.713106) (width 0.2) (layer "F.Cu") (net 11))
 (segment (start 115.551 119.713106) (end 115.311894 119.474) (width 0.2) (layer "F.Cu") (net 11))
 (segment (start 71.569686 135.441) (end 72.730314 135.441) (width 0.2) (layer "F.Cu") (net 11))
 (segment (start 45.349 101.191) (end 45.349 103.05676) (width 0.2) (layer "F.Cu") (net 11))
 (segment (start 46.5 100.04) (end 45.349 101.191) (width 0.2) (layer "F.Cu") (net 11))
 (segment (start 73.551 133.459686) (end 72.730314 132.639) (width 0.2) (layer "F.Cu") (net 11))
 (segment (start 74.986184 138.931) (end 76.933816 138.931) (width 0.2) (layer "F.Cu") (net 11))
 (segment (start 71.569686 132.639) (end 70.749 133.459686) (width 0.2) (layer "F.Cu") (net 11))
 (segment (start 108.069686 133.139) (end 107.569686 133.639) (width 0.2) (layer "F.Cu") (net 11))
 (segment (start 73.609 137.553816) (end 74.986184 138.931) (width 0.2) (layer "F.Cu") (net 11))
 (segment (start 107.249 134.441) (end 107.249 135.120314) (width 0.2) (layer "F.Cu") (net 11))
 (segment (start 115.351 130.599) (end 115.351 120.486894) (width 0.2) (layer "F.Cu") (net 11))
 (segment (start 114.419686 130.599) (end 113.599 131.419686) (width 0.2) (layer "F.Cu") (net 11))
 (segment (start 74.774184 134.441) (end 73.609 135.606184) (width 0.2) (layer "F.Cu") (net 11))
 (segment (start 116.802 132.746414) (end 116.802 118.802) (width 0.2) (layer "F.Cu") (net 11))
 (segment (start 110.051 135.120314) (end 110.051 134.441) (width 0.2) (layer "F.Cu") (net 11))
 (segment (start 114.349 119.713106) (end 114.349 120.286894) (width 0.2) (layer "F.Cu") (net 11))
 (segment (start 78.311 135.606184) (end 77.145816 134.441) (width 0.2) (layer "F.Cu") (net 11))
 (segment (start 73.551 133.639) (end 73.551 133.459686) (width 0.2) (layer "F.Cu") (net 11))
 (segment (start 77.145816 134.441) (end 107.249 134.441) (width 0.2) (layer "F.Cu") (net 11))
 (segment (start 78.311 137.553816) (end 78.311 135.606184) (width 0.2) (layer "F.Cu") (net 11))
 (segment (start 114.419686 133.401) (end 115.013214 133.401) (width 0.2) (layer "F.Cu") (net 11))
 (segment (start 77.85 94.96) (end 77.85 75.15) (width 0.2) (layer "F.Cu") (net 1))
 (segment (start 77.85 75.15) (end 78 75) (width 0.2) (layer "F.Cu") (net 1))
 (segment (start 74.606 74.474) (end 46.5 102.58) (width 0.2) (layer "F.Cu") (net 4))
 (segment (start 104.46 96.139) (end 103.639314 96.959686) (width 0.2) (layer "F.Cu") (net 4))
 (segment (start 80.1 75) (end 79.112106 75) (width 0.2) (layer "F.Cu") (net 4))
 (segment (start 124.551 96.959686) (end 123.730314 96.139) (width 0.2) (layer "F.Cu") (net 4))
 (segment (start 79 75.112106) (end 78.361894 74.474) (width 0.2) (layer "F.Cu") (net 4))
 (segment (start 117.651 120) (end 124.551 113.1) (width 0.2) (layer "F.Cu") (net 4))
 (segment (start 118.0755 119.5755) (end 117.651 120) (width 0.2) (layer "F.Cu") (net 4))
 (segment (start 124.551 113.1) (end 118.0755 119.5755) (width 0.2) (layer "F.Cu") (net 4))
 (segment (start 79.112106 75) (end 79 75.112106) (width 0.2) (layer "F.Cu") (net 4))
 (segment (start 100.459686 96.959686) (end 79 75.5) (width 0.2) (layer "F.Cu") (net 4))
 (segment (start 103.639314 96.959686) (end 100.459686 96.959686) (width 0.2) (layer "F.Cu") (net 4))
 (segment (start 124.551 113.1) (end 124.551 96.959686) (width 0.2) (layer "F.Cu") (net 4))
 (segment (start 78.361894 74.474) (end 74.606 74.474) (width 0.2) (layer "F.Cu") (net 4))
 (segment (start 79 75.112106) (end 79 75.5) (width 0.2) (layer "F.Cu") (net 4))
 (segment (start 123.730314 96.139) (end 104.46 96.139) (width 0.2) (layer "F.Cu") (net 4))
 (segment (start 46.5 105.12) (end 59.354 117.974) (width 0.2) (layer "F.Cu") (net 8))
 (segment (start 59.354 117.974) (end 79.974 117.974) (width 0.2) (layer "F.Cu") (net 8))
 (segment (start 80.05 118) (end 80.55 118.5) (width 0.2) (layer "F.Cu") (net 8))
 (segment (start 79.974 117.974) (end 80 118) (width 0.2) (layer "F.Cu") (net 8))
 (segment (start 80 118) (end 80.05 118) (width 0.2) (layer "F.Cu") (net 8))
 (segment (start 78.5 118.55) (end 78.45 118.5) (width 0.2) (layer "F.Cu") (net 5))
 (segment (start 78.5 131.5) (end 78.5 118.55) (width 0.2) (layer "F.Cu") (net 5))
 (segment (start 123.15 97.54) (end 123.15 100.50847) (width 0.2) (layer "F.Cu") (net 2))
 (segment (start 116.401 118.5) (end 116.401 132.580314) (width 0.2) (layer "F.Cu") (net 2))
 (segment (start 71.5 97.5) (end 123.11 97.5) (width 0.2) (layer "F.Cu") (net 2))
 (segment (start 116.401 107.25747) (end 116.401 111) (width 0.2) (layer "F.Cu") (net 2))
 (segment (start 114.941314 134.04) (end 72.15 134.04) (width 0.2) (layer "F.Cu") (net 2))
 (segment (start 123.11 97.5) (end 123.15 97.54) (width 0.2) (layer "F.Cu") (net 2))
 (segment (start 116.401 132.580314) (end 114.941314 134.04) (width 0.2) (layer "F.Cu") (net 2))
 (segment (start 116.401 111) (end 116.401 118.5) (width 0.2) (layer "F.Cu") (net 2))
 (segment (start 123.15 100.50847) (end 116.401 107.25747) (width 0.2) (layer "F.Cu") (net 2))
 (segment (start 97.11 97.5) (end 97.15 97.54) (width 0.2) (layer "F.Cu") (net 2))
 (segment (start 71.5 97.5) (end 97.11 97.5) (width 0.2) (layer "F.Cu") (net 2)))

